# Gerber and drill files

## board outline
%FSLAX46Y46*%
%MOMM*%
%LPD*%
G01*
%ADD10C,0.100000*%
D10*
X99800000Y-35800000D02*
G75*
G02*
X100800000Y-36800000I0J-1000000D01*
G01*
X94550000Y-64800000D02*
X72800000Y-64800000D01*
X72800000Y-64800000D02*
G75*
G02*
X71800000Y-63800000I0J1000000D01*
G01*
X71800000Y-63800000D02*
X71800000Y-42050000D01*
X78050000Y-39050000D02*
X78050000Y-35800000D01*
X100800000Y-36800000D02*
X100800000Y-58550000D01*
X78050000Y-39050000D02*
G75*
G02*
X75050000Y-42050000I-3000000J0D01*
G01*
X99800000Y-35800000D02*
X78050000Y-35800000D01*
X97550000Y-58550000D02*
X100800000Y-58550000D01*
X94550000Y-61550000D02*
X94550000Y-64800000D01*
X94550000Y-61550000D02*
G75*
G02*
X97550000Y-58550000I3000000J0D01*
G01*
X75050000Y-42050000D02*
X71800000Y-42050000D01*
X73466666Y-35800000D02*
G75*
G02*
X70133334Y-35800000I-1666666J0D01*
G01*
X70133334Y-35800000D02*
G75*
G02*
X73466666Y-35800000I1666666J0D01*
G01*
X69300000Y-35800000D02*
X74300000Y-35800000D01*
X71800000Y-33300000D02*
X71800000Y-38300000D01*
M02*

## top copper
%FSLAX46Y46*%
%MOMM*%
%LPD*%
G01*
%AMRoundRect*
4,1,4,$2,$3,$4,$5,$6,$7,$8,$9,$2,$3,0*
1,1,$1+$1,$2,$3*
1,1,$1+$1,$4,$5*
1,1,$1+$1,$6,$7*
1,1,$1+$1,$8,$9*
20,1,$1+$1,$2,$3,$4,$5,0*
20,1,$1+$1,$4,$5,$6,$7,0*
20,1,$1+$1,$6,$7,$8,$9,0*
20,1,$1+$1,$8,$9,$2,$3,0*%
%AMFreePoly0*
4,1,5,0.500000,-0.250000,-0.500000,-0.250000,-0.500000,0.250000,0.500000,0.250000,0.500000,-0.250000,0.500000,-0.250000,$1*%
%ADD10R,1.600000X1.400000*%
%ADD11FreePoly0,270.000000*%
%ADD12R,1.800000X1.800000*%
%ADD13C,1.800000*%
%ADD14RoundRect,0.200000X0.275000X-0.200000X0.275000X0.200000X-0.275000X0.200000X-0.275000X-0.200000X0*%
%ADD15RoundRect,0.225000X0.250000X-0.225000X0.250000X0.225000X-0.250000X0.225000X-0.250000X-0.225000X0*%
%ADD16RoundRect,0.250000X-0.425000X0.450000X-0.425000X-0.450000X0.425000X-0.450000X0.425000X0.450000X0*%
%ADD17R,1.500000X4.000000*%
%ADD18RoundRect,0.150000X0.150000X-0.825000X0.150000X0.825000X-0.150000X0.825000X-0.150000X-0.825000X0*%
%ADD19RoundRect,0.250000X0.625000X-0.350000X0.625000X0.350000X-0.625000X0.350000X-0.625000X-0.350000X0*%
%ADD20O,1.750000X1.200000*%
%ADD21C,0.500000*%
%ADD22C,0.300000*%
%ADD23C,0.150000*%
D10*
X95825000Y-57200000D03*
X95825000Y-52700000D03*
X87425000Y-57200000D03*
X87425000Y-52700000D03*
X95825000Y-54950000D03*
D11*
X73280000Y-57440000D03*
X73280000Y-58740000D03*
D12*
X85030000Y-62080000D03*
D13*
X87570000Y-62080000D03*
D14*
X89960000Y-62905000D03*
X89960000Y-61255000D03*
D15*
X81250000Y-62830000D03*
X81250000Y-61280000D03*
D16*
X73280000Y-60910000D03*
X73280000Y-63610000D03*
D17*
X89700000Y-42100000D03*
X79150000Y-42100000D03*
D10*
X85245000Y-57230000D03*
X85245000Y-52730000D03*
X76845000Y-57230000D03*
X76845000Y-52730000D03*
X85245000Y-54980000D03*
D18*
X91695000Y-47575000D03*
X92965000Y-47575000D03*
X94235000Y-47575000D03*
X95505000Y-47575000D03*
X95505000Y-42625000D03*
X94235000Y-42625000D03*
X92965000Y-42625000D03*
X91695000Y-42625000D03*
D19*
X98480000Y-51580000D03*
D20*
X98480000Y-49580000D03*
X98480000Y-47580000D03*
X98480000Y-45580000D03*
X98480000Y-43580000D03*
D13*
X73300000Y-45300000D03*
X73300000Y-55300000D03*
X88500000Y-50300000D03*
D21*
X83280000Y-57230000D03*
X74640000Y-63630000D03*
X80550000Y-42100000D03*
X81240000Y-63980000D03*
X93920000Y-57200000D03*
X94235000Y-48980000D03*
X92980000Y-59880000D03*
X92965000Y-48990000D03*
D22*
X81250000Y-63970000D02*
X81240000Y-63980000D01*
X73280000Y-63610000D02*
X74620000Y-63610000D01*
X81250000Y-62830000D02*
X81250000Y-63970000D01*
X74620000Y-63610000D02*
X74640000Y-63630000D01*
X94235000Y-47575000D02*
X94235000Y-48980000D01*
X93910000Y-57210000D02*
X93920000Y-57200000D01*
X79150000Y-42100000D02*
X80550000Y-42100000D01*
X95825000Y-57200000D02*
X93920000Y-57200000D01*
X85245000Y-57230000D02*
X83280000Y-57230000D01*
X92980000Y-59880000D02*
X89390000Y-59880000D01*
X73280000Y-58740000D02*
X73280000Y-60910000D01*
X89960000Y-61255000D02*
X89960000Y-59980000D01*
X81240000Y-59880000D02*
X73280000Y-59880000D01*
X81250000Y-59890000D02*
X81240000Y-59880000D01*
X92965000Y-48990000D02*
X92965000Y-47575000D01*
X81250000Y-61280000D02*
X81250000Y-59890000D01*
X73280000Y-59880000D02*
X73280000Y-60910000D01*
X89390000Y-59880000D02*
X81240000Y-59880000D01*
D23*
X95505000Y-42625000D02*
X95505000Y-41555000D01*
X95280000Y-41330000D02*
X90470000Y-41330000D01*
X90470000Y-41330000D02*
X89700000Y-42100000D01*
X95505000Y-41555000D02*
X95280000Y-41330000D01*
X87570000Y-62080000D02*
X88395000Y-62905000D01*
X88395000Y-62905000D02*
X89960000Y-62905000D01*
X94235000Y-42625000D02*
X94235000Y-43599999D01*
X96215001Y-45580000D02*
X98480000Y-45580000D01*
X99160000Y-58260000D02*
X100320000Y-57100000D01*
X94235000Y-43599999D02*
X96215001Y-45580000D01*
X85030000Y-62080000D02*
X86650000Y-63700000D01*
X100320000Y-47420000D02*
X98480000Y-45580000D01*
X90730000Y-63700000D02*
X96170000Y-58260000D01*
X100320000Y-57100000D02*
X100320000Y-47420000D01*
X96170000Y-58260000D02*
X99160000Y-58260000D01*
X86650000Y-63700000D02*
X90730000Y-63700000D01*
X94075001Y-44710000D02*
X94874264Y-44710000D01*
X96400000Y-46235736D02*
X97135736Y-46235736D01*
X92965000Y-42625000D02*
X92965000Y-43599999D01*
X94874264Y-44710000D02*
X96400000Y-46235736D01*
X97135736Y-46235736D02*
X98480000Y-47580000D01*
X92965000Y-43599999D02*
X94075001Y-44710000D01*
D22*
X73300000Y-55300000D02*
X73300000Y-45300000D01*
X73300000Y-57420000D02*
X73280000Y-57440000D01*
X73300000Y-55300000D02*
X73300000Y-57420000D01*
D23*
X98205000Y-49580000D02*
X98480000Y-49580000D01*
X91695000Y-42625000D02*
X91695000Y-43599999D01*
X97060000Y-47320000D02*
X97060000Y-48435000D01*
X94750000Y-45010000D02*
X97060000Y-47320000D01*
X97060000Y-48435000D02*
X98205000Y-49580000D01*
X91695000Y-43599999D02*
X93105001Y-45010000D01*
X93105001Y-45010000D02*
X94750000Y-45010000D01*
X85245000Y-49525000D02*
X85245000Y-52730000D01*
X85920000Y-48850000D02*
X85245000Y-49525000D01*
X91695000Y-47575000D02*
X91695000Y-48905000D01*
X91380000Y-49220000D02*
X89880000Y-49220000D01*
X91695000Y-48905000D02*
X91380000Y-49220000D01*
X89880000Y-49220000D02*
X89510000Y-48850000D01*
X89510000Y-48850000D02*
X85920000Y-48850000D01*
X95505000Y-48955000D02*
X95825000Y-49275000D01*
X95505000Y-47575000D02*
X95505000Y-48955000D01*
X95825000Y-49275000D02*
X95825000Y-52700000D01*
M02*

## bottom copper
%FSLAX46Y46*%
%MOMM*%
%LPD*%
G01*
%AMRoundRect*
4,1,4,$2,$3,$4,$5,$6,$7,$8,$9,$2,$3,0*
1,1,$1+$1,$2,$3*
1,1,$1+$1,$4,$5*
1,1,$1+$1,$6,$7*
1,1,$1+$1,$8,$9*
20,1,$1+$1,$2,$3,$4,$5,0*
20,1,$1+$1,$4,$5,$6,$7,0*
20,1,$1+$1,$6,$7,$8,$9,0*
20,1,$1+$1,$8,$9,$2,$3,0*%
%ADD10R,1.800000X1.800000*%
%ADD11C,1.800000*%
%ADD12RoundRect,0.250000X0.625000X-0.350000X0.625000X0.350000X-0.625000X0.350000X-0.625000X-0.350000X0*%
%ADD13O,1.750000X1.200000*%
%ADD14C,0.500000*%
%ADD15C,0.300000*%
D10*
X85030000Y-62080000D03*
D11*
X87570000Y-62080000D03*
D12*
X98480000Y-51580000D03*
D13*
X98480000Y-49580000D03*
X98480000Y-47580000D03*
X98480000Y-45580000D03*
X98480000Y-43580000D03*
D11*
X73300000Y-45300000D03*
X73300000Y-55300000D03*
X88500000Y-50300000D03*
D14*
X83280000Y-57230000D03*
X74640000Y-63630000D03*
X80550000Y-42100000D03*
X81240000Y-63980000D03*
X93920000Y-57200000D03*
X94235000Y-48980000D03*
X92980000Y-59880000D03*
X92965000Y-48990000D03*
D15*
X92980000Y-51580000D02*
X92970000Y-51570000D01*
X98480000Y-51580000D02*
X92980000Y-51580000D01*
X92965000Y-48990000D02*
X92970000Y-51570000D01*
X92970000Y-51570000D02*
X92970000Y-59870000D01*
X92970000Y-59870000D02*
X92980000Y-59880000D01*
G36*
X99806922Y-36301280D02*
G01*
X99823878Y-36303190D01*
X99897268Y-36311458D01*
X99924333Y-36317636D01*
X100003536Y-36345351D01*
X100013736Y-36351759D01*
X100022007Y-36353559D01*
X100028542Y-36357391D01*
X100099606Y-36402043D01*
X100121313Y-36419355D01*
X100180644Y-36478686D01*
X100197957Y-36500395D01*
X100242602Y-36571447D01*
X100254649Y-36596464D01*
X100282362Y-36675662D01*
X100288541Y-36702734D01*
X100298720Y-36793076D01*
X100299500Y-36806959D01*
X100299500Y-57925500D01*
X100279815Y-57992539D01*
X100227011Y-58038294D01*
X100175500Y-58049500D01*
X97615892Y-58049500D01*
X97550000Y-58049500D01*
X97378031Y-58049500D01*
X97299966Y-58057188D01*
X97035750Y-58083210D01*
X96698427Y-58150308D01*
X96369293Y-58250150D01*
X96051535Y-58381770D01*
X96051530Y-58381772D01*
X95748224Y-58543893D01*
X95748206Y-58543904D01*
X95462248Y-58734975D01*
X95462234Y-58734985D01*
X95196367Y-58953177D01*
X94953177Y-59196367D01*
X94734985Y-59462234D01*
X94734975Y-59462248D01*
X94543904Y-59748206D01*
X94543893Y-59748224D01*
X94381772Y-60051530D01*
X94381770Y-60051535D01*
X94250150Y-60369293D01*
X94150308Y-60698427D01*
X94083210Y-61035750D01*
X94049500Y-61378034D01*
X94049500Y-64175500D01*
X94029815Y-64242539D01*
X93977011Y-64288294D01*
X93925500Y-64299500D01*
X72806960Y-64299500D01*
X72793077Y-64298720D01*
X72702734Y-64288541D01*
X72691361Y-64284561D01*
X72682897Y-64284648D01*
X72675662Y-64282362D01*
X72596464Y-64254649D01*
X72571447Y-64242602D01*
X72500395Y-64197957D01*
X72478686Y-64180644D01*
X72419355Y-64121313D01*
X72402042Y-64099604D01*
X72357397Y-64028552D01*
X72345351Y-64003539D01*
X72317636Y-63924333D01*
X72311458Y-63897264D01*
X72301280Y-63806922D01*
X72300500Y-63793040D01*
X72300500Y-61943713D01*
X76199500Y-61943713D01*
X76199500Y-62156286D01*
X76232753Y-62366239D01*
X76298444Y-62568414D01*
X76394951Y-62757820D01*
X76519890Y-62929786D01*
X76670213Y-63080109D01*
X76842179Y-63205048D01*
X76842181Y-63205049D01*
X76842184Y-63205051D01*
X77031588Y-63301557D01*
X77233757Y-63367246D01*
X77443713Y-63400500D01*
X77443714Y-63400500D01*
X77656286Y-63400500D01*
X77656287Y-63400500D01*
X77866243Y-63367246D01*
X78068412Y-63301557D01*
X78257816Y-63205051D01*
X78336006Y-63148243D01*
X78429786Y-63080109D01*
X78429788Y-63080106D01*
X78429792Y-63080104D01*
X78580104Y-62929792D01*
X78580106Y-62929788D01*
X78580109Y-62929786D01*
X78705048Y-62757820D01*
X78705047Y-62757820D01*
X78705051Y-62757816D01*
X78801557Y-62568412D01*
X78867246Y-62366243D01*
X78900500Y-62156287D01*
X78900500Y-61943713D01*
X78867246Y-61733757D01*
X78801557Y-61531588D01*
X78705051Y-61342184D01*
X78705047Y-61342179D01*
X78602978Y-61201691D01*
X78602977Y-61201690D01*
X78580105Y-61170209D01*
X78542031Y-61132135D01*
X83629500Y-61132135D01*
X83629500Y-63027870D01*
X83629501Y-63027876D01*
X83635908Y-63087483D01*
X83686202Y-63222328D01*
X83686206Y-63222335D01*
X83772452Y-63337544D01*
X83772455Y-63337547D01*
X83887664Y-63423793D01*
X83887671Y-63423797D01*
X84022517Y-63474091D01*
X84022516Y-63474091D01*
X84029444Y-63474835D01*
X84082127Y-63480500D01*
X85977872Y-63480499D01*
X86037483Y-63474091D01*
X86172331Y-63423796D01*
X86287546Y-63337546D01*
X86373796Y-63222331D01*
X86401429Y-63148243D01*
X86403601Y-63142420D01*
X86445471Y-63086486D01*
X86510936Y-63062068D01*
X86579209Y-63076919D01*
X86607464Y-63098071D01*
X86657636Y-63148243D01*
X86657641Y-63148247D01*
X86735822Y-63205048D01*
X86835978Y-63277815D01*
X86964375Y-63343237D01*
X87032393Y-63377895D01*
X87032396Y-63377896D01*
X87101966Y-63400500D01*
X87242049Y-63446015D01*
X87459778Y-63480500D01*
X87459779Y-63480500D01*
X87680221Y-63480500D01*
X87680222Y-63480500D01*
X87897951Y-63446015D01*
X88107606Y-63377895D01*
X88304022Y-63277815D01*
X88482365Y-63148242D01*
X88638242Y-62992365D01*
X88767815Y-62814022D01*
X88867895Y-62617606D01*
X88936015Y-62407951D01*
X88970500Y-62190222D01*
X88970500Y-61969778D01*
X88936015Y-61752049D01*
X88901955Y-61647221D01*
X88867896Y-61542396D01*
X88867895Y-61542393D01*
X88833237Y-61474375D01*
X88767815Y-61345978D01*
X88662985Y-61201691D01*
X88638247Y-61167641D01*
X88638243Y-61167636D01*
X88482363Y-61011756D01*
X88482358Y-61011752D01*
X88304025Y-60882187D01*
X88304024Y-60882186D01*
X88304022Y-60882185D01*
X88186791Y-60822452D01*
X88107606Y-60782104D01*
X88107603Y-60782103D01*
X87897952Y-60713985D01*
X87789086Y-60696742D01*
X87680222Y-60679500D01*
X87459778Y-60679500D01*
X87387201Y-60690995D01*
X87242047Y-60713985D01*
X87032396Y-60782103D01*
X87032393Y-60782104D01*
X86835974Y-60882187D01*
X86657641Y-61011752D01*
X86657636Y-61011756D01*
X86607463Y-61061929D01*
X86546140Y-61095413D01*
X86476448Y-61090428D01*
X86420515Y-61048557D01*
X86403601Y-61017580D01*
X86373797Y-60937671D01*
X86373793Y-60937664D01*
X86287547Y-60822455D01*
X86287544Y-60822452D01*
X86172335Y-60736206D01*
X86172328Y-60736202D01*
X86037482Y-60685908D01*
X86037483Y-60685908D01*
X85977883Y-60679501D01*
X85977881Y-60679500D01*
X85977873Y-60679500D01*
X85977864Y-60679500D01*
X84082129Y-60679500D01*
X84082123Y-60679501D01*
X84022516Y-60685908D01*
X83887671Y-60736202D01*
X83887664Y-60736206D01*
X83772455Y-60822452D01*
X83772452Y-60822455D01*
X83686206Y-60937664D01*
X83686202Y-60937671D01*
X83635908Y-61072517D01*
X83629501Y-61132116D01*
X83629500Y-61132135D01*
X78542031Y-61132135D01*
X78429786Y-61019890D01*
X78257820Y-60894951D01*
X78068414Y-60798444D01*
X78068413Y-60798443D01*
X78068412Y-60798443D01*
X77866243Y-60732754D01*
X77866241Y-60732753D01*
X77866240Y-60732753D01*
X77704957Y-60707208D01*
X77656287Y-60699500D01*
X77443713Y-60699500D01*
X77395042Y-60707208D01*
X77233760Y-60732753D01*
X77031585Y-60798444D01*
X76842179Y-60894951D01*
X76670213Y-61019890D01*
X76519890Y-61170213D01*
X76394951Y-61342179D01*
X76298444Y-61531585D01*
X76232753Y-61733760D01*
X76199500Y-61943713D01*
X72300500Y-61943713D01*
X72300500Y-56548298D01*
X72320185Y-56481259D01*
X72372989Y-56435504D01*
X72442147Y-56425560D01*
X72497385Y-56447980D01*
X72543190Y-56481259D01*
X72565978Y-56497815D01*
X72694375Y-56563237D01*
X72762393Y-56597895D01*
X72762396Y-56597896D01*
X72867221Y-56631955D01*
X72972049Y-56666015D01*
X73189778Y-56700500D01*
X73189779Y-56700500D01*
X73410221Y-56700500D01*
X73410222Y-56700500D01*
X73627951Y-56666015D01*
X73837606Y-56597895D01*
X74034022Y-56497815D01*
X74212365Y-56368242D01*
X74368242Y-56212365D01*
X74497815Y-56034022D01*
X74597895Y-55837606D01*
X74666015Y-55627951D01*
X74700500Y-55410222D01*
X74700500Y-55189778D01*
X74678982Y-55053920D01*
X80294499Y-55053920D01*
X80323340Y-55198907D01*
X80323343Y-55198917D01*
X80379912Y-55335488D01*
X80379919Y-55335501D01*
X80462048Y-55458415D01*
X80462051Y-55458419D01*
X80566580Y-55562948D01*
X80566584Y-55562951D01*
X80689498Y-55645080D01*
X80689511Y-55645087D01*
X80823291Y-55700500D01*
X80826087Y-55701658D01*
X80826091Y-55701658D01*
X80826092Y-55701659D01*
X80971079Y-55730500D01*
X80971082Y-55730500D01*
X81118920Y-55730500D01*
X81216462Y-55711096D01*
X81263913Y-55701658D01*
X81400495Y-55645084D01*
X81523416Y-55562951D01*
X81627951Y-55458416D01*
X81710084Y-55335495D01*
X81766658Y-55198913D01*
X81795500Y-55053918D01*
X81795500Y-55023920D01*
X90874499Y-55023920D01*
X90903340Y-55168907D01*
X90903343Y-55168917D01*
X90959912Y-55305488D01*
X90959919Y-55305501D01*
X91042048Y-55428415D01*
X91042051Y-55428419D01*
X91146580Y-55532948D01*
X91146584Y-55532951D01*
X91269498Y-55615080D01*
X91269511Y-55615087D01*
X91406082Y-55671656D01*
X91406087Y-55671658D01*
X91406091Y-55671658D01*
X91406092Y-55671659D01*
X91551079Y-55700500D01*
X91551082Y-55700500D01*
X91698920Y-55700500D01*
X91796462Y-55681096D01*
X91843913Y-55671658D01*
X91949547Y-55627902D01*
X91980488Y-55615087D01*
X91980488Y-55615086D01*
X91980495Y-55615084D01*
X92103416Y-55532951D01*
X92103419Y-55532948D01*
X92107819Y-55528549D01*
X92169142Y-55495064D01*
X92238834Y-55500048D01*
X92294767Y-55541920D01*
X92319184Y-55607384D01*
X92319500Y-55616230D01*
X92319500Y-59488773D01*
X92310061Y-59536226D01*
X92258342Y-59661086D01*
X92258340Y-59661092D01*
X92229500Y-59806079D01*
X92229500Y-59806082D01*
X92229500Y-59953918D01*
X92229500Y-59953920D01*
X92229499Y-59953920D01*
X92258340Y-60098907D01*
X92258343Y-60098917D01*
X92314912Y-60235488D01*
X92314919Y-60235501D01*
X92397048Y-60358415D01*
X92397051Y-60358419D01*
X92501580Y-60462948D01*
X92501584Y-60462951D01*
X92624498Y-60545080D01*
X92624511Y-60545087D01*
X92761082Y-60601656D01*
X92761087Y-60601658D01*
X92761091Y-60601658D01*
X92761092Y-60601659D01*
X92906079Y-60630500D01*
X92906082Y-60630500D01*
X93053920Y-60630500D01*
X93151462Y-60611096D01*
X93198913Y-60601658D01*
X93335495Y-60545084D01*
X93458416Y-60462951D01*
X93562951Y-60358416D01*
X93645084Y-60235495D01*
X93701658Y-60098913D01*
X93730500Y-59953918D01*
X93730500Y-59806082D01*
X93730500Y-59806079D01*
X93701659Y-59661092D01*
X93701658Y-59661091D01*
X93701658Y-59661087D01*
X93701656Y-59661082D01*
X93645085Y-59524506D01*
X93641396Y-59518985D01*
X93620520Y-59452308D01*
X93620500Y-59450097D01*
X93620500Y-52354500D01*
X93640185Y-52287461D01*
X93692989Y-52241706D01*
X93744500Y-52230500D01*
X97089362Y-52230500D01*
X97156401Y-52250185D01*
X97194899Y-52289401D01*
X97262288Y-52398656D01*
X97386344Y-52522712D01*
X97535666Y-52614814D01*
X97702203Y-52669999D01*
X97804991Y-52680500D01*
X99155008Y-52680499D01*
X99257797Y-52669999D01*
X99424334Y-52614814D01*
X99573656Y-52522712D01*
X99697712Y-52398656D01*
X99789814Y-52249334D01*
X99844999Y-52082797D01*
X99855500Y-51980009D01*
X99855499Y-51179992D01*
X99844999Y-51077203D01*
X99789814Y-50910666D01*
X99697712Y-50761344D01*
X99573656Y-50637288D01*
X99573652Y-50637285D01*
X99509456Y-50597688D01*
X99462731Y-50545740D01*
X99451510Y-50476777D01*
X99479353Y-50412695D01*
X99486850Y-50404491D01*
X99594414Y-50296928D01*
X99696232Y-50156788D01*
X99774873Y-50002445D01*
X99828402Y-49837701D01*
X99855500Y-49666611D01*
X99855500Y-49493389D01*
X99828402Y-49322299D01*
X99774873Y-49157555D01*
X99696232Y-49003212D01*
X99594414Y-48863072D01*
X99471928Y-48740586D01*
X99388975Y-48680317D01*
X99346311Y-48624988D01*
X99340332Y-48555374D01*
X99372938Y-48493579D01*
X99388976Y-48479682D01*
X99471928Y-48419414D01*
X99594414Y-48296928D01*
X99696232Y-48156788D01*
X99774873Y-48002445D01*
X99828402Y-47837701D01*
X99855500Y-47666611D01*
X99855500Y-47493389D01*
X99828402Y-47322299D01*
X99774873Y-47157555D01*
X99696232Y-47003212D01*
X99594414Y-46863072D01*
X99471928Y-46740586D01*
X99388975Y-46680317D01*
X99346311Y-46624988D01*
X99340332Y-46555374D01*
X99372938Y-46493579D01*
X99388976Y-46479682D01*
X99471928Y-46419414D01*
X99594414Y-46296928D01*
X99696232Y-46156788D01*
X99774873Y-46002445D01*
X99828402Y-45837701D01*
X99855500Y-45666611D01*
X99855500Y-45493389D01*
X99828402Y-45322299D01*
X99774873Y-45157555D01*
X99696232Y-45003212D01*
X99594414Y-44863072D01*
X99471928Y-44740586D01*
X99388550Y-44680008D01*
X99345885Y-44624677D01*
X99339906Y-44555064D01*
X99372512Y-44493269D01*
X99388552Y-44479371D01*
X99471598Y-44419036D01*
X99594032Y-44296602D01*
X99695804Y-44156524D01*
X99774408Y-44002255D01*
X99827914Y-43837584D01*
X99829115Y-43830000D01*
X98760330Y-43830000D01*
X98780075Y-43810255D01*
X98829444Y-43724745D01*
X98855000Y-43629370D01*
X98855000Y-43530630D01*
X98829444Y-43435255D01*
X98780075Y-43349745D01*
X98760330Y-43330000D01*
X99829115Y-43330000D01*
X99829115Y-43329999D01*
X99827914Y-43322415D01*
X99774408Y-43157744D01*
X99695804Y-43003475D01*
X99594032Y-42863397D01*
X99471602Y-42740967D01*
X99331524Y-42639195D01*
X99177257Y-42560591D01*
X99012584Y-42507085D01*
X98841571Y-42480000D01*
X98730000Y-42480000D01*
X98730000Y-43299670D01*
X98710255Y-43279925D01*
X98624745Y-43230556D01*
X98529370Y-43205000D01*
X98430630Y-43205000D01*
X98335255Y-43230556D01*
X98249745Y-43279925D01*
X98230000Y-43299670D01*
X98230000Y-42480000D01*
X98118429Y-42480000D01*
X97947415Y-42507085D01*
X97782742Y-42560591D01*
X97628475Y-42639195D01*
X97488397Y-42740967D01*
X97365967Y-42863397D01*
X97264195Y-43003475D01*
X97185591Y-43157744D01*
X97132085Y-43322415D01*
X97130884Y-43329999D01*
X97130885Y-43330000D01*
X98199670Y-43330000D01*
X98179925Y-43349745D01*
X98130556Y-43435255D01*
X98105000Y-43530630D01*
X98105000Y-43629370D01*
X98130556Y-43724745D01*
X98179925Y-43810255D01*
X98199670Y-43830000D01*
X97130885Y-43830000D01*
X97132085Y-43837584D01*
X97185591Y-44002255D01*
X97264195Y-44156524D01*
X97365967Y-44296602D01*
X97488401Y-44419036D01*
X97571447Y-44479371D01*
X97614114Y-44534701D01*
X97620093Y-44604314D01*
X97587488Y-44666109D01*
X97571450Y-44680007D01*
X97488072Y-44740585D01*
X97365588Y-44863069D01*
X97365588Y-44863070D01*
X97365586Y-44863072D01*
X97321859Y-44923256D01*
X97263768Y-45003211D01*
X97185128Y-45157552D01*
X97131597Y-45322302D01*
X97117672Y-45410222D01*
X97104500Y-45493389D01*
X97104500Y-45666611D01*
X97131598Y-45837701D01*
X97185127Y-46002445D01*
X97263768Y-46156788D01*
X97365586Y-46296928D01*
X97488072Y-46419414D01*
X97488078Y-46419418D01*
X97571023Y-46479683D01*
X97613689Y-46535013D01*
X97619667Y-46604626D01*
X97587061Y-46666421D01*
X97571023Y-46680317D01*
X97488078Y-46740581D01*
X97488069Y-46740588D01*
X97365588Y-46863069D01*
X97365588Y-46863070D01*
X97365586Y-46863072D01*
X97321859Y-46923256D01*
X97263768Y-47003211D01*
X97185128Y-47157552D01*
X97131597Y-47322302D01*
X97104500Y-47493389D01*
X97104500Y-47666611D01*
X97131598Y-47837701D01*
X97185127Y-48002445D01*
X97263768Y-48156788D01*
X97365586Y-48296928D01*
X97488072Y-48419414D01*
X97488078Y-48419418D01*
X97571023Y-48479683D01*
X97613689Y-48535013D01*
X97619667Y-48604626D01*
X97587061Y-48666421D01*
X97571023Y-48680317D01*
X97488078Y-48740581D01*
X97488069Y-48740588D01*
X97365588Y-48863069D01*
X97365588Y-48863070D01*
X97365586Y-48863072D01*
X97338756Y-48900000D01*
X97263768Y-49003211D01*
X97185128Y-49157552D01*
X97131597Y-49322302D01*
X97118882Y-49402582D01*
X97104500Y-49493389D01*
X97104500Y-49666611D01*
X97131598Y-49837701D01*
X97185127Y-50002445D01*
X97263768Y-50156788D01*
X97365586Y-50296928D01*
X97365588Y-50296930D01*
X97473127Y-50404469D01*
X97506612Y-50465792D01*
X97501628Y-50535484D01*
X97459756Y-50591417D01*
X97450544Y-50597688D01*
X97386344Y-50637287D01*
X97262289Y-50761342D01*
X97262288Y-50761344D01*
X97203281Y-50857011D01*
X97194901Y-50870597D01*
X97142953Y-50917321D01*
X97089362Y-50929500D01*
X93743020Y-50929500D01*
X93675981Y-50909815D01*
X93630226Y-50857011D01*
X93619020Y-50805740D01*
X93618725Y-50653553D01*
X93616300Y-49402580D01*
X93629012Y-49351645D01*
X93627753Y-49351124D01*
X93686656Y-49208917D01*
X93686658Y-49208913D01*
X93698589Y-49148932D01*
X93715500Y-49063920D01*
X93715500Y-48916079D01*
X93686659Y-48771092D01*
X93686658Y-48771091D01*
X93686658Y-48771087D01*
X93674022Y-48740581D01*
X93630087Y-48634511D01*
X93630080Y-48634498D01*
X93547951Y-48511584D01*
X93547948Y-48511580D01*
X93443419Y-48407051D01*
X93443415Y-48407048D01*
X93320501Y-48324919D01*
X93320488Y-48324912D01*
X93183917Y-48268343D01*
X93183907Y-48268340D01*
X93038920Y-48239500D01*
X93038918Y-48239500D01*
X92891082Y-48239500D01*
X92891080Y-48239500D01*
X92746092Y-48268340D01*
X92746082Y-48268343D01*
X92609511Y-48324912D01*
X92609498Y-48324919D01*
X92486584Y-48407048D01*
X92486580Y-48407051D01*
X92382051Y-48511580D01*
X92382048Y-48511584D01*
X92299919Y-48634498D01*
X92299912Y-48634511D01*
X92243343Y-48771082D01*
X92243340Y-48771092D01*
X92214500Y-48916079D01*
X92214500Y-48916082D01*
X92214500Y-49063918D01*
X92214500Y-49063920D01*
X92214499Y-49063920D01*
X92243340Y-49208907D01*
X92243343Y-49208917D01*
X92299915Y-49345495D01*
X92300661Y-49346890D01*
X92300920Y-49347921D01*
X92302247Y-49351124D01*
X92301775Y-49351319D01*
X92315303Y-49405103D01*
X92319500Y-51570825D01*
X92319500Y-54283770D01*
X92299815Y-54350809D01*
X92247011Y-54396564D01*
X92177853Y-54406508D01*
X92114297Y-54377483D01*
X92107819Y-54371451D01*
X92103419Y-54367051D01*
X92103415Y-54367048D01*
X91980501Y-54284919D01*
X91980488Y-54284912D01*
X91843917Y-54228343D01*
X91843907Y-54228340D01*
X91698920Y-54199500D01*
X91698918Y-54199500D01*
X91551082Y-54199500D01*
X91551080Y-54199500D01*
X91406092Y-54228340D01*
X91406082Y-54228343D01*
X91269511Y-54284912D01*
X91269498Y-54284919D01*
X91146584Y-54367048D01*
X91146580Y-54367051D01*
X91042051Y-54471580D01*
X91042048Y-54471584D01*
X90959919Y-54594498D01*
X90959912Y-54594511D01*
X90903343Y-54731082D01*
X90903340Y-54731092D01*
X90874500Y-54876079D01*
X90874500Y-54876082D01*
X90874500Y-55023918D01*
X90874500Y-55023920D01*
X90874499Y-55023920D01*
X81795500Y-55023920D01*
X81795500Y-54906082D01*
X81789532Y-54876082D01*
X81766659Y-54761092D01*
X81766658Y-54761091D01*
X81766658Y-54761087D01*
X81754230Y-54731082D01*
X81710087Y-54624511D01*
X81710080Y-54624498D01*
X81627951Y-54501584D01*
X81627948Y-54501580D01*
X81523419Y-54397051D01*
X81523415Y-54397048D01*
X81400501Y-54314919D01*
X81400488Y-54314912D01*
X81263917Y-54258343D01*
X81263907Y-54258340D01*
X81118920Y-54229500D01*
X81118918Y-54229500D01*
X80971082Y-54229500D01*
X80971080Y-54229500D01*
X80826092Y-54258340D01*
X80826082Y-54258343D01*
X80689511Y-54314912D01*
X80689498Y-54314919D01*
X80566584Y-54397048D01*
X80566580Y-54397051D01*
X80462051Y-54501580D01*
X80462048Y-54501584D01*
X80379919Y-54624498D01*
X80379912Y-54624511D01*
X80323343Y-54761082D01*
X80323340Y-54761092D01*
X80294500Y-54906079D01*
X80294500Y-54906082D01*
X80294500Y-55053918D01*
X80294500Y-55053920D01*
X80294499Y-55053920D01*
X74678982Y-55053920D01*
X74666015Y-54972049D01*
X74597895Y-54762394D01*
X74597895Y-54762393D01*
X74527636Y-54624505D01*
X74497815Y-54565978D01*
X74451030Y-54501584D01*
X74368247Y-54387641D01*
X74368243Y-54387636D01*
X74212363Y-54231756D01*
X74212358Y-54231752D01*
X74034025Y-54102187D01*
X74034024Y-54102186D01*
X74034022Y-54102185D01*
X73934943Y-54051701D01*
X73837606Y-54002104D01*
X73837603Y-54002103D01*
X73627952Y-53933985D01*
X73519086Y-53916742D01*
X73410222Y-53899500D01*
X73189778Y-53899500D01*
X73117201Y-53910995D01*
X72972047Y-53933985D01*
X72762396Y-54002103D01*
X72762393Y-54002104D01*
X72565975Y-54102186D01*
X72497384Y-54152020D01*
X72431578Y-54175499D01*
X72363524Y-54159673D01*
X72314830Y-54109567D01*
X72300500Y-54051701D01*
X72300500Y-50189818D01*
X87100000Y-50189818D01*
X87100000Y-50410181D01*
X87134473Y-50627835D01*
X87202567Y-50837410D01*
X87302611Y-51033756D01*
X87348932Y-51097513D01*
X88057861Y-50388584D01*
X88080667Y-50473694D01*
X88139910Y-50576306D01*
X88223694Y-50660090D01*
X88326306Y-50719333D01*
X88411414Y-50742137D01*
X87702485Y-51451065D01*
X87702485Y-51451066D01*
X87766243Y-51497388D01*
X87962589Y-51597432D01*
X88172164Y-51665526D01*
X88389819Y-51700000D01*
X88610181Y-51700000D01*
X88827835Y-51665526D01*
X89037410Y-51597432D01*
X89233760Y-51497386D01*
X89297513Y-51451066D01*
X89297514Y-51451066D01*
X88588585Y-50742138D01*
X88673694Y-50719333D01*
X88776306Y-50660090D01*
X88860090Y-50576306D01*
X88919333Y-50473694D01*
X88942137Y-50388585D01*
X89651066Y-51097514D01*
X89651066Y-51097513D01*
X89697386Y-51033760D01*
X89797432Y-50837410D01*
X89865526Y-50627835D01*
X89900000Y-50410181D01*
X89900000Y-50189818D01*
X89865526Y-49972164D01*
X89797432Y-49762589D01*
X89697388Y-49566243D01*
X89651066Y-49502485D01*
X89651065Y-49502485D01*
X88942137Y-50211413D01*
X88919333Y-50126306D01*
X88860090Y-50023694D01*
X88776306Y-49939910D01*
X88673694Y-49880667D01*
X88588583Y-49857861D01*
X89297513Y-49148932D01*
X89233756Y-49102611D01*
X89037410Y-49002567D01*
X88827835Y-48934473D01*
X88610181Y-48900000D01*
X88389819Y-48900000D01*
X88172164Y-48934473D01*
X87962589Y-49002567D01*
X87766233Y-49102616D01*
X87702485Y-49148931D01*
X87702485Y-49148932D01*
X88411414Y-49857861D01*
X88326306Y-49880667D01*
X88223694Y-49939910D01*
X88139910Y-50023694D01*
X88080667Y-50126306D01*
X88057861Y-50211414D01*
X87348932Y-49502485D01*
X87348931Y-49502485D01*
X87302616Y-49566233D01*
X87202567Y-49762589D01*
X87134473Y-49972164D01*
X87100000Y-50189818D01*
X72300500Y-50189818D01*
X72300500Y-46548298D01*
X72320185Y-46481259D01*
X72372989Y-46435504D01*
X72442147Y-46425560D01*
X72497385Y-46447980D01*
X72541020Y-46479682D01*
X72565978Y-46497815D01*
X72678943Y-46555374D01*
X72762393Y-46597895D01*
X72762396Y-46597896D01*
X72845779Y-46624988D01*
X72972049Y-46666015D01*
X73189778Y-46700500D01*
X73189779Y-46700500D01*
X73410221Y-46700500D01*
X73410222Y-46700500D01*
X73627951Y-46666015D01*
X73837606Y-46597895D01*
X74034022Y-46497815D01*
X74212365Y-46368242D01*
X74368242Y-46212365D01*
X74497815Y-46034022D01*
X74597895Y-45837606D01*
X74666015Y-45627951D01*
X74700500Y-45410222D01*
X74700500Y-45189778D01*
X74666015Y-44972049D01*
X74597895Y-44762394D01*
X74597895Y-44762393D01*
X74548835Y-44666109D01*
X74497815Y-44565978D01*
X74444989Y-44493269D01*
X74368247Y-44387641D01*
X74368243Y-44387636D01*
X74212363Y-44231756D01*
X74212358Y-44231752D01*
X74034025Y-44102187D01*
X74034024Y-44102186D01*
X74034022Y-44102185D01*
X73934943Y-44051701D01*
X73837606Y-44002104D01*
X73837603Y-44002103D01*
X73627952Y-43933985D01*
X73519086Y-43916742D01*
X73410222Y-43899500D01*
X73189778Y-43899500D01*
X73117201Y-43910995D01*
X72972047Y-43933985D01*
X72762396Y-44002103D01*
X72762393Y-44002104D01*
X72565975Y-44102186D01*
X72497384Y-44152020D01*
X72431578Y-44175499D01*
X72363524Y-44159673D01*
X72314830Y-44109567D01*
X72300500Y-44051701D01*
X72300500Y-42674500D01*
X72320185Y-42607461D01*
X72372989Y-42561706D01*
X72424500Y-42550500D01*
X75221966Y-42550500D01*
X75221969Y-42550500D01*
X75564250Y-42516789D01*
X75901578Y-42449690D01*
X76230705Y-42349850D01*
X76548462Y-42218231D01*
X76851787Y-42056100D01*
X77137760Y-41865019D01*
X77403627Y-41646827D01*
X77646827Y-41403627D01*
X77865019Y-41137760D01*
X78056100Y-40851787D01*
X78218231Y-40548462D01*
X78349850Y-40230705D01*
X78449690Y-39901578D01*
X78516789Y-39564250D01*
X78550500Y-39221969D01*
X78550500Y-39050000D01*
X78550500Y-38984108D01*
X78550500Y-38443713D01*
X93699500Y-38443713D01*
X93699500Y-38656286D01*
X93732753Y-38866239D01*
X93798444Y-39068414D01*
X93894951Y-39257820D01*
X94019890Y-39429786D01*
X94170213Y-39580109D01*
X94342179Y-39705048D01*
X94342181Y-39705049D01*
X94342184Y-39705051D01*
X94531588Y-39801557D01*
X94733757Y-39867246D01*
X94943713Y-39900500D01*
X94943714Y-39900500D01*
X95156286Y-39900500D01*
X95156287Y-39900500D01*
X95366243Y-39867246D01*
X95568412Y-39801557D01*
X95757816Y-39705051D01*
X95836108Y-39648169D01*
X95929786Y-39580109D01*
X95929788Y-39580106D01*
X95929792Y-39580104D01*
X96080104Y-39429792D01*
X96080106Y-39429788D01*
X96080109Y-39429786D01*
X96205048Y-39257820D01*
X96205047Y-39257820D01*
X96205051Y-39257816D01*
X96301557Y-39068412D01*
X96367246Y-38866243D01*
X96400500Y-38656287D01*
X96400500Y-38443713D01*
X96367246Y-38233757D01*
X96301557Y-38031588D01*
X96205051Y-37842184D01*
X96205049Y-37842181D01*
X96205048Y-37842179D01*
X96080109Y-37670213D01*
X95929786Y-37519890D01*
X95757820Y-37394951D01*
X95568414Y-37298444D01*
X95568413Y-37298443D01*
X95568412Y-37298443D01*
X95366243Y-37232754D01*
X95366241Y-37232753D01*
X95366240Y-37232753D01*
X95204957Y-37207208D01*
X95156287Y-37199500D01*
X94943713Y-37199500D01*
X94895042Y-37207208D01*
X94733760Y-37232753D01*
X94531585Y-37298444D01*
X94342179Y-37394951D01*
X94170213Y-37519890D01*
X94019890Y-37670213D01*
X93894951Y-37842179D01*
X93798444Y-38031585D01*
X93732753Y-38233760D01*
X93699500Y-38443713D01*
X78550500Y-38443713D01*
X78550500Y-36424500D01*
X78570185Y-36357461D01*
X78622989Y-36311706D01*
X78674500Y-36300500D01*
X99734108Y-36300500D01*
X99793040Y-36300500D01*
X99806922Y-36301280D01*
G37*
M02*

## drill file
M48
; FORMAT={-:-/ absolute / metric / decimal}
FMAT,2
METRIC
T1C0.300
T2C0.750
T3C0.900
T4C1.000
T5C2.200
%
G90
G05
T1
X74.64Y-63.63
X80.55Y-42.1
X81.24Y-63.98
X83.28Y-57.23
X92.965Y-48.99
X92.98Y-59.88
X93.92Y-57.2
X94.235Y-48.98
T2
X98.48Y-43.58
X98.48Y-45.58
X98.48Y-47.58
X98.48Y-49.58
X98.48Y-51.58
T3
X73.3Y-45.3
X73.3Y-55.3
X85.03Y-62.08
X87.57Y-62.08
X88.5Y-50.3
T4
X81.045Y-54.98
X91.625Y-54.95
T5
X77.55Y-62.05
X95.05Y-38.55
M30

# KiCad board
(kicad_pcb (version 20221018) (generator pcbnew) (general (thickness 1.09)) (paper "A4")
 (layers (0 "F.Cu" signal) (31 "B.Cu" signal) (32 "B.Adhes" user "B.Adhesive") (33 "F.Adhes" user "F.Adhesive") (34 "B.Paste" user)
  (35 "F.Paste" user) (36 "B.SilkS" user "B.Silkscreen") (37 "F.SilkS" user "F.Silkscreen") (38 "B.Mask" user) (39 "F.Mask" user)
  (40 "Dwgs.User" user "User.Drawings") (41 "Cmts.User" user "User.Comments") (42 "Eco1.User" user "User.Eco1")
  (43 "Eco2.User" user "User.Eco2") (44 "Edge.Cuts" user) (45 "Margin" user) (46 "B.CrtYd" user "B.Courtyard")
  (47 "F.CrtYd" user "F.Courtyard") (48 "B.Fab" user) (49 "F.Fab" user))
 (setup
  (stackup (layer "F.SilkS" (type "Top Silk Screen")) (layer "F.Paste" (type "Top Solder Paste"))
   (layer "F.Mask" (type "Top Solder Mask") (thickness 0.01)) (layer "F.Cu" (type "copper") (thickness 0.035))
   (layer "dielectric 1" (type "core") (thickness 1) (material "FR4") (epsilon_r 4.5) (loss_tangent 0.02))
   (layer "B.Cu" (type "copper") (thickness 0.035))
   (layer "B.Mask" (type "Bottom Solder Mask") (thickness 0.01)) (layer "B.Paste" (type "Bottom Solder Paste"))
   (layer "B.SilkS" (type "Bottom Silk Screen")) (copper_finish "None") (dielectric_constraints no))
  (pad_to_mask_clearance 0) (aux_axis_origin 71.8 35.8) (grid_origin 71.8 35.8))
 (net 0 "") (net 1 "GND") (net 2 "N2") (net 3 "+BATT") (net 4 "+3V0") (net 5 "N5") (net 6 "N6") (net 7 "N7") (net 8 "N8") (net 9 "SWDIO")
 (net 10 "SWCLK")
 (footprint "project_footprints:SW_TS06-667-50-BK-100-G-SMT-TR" (layer "F.Cu") (at 91.625 54.95 180)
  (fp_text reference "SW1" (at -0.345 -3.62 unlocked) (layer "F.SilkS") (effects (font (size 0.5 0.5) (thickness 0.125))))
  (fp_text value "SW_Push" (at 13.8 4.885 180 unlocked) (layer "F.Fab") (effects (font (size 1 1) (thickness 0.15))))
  (pad "1" smd rect (at -4.2 -2.25 180) (size 1.6 1.4) (layers "F.Cu" "F.Paste" "F.Mask") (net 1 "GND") (solder_mask_margin 0.102))
  (pad "2" smd rect (at -4.2 2.25 180) (size 1.6 1.4) (layers "F.Cu" "F.Paste" "F.Mask") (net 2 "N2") (solder_mask_margin 0.102))
  (pad "3" smd rect (at 4.2 -2.25 180) (size 1.6 1.4) (layers "F.Cu" "F.Paste" "F.Mask") (solder_mask_margin 0.102))
  (pad "4" smd rect (at 4.2 2.25 180) (size 1.6 1.4) (layers "F.Cu" "F.Paste" "F.Mask") (solder_mask_margin 0.102))
  (pad "5" smd rect (at -4.2 0 180) (size 1.6 1.4) (layers "F.Cu" "F.Paste" "F.Mask") (solder_mask_margin 0.102)))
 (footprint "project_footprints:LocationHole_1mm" (layer "F.Cu") (at 81.045 54.98)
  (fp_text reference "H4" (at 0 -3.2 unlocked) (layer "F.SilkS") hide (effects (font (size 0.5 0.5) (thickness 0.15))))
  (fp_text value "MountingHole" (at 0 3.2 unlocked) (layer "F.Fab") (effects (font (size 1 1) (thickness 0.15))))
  (pad "" np_thru_hole circle (at 0 0) (size 1 1) (drill 1) (layers "F&B.Cu" "*.Mask")))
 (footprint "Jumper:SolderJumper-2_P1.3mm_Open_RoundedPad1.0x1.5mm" (layer "F.Cu") (at 73.28 58.09 -90) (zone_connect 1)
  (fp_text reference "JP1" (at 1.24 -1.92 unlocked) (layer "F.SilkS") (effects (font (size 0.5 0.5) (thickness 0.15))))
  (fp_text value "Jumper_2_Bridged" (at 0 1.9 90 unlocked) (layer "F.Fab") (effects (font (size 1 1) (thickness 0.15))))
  (pad "1" smd custom (at -0.65 0 270) (size 1 0.5) (layers "F.Cu" "F.Mask") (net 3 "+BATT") (zone_connect 2) (thermal_bridge_angle 45)
   (options (clearance outline) (anchor rect)) (primitives))
  (pad "2" smd custom (at 0.65 0 270) (size 1 0.5) (layers "F.Cu" "F.Mask") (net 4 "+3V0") (zone_connect 2) (thermal_bridge_angle 45)
   (options (clearance outline) (anchor rect)) (primitives)))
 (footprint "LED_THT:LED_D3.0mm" (layer "F.Cu") (at 85.03 62.08)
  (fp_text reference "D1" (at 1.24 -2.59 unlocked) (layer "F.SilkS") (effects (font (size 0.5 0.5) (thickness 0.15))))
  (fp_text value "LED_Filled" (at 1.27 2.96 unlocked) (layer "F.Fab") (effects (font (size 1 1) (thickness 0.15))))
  (pad "1" thru_hole rect (at 0 0) (size 1.8 1.8) (drill 0.9) (layers "*.Cu" "*.Mask") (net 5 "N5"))
  (pad "2" thru_hole circle (at 2.54 0) (size 1.8 1.8) (drill 0.9) (layers "*.Cu" "*.Mask") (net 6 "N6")))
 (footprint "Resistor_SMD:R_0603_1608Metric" (layer "F.Cu") (at 89.96 62.08 90)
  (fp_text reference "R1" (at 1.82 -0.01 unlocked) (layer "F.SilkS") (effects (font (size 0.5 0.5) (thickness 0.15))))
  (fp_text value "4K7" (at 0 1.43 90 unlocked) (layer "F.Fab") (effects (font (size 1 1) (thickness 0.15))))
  (pad "1" smd roundrect (at -0.825 0 90) (size 0.8 0.95) (layers "F.Cu" "F.Paste" "F.Mask") (roundrect_rratio 0.25) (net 6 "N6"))
  (pad "2" smd roundrect (at 0.825 0 90) (size 0.8 0.95) (layers "F.Cu" "F.Paste" "F.Mask") (roundrect_rratio 0.25) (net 4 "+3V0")))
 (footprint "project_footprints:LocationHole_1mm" (layer "F.Cu") (at 91.625 54.95)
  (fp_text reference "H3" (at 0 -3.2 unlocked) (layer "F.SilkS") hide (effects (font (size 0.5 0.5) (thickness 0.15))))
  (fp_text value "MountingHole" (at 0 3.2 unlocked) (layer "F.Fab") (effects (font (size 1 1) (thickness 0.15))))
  (pad "" np_thru_hole circle (at 0 0) (size 1 1) (drill 1) (layers "F&B.Cu" "*.Mask")))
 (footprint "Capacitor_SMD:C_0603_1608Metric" (layer "F.Cu") (at 81.25 62.055 90)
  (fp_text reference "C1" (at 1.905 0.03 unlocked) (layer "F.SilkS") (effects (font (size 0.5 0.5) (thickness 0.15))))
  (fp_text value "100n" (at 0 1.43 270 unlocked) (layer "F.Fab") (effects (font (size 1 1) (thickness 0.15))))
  (pad "1" smd roundrect (at -0.775 0 90) (size 0.9 0.95) (layers "F.Cu" "F.Paste" "F.Mask") (roundrect_rratio 0.25) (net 1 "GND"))
  (pad "2" smd roundrect (at 0.775 0 90) (size 0.9 0.95) (layers "F.Cu" "F.Paste" "F.Mask") (roundrect_rratio 0.25) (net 4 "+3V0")))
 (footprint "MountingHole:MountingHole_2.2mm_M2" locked (layer "F.Cu") (at 77.55 62.05)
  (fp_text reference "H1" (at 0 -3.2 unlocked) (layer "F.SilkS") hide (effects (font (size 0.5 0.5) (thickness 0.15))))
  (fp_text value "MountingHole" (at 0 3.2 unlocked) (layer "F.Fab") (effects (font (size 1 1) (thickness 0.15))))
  (pad "" np_thru_hole circle locked (at 0 0) (size 2.2 2.2) (drill 2.2) (layers "*.Cu" "*.Mask")))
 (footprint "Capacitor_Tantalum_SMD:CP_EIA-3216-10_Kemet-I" (layer "F.Cu") (at 73.28 62.26 -90)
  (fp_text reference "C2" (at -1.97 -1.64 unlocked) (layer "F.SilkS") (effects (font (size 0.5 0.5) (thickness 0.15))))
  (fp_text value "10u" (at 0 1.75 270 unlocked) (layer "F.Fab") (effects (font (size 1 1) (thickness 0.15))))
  (pad "1" smd roundrect (at -1.35 0 270) (size 1.4 1.35) (layers "F.Cu" "F.Paste" "F.Mask") (roundrect_rratio 0.1851851852) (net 4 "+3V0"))
  (pad "2" smd roundrect (at 1.35 0 270) (size 1.4 1.35) (layers "F.Cu" "F.Paste" "F.Mask") (roundrect_rratio 0.1851851852) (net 1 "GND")))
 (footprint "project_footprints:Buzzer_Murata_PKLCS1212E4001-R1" (layer "F.Cu") (at 84.4 42.1 180)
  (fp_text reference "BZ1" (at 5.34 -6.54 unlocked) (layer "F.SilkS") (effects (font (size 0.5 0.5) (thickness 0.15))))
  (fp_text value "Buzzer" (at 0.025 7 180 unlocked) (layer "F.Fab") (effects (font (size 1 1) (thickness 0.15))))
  (pad "1" smd rect (at -5.3 0 180) (size 1.5 4) (layers "F.Cu" "F.Paste" "F.Mask") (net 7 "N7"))
  (pad "2" smd rect (at 5.25 0 180) (size 1.5 4) (layers "F.Cu" "F.Paste" "F.Mask") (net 1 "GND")))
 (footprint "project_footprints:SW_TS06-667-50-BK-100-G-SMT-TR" (layer "F.Cu") (at 81.045 54.98 180)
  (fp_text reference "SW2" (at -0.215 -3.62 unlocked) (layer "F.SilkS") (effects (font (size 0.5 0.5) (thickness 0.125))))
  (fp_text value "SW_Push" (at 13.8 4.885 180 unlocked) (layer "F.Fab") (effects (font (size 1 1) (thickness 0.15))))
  (pad "1" smd rect (at -4.2 -2.25 180) (size 1.6 1.4) (layers "F.Cu" "F.Paste" "F.Mask") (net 1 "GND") (solder_mask_margin 0.102))
  (pad "2" smd rect (at -4.2 2.25 180) (size 1.6 1.4) (layers "F.Cu" "F.Paste" "F.Mask") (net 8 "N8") (solder_mask_margin 0.102))
  (pad "3" smd rect (at 4.2 -2.25 180) (size 1.6 1.4) (layers "F.Cu" "F.Paste" "F.Mask") (solder_mask_margin 0.102))
  (pad "4" smd rect (at 4.2 2.25 180) (size 1.6 1.4) (layers "F.Cu" "F.Paste" "F.Mask") (solder_mask_margin 0.102))
  (pad "5" smd rect (at -4.2 0 180) (size 1.6 1.4) (layers "F.Cu" "F.Paste" "F.Mask") (solder_mask_margin 0.102)))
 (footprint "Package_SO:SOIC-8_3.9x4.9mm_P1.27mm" (layer "F.Cu") (at 93.6 45.1 90)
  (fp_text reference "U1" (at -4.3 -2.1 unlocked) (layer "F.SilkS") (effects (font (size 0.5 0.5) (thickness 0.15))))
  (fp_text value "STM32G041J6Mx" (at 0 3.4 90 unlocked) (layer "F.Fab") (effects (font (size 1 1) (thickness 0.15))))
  (pad "1" smd roundrect (at -2.475 -1.905 90) (size 1.95 0.6) (layers "F.Cu" "F.Paste" "F.Mask") (roundrect_rratio 0.25) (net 8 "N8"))
  (pad "2" smd roundrect (at -2.475 -0.635 90) (size 1.95 0.6) (layers "F.Cu" "F.Paste" "F.Mask") (roundrect_rratio 0.25) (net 4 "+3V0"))
  (pad "3" smd roundrect (at -2.475 0.635 90) (size 1.95 0.6) (layers "F.Cu" "F.Paste" "F.Mask") (roundrect_rratio 0.25) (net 1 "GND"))
  (pad "4" smd roundrect (at -2.475 1.905 90) (size 1.95 0.6) (layers "F.Cu" "F.Paste" "F.Mask") (roundrect_rratio 0.25) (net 2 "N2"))
  (pad "5" smd roundrect (at 2.475 1.905 90) (size 1.95 0.6) (layers "F.Cu" "F.Paste" "F.Mask") (roundrect_rratio 0.25) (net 7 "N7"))
  (pad "6" smd roundrect (at 2.475 0.635 90) (size 1.95 0.6) (layers "F.Cu" "F.Paste" "F.Mask") (roundrect_rratio 0.25) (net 5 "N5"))
  (pad "7" smd roundrect (at 2.475 -0.635 90) (size 1.95 0.6) (layers "F.Cu" "F.Paste" "F.Mask") (roundrect_rratio 0.25) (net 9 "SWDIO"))
  (pad "8" smd roundrect (at 2.475 -1.905 90) (size 1.95 0.6) (layers "F.Cu" "F.Paste" "F.Mask") (roundrect_rratio 0.25) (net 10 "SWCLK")))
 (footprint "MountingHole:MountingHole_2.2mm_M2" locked (layer "F.Cu") (at 95.05 38.55)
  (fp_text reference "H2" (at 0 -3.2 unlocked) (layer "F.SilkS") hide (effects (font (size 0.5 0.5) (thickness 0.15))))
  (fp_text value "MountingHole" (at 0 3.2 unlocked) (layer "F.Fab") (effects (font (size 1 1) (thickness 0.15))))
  (pad "" np_thru_hole circle locked (at 0 0) (size 2.2 2.2) (drill 2.2) (layers "*.Cu" "*.Mask")))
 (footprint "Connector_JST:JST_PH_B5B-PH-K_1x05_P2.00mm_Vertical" (layer "B.Cu") (at 98.48 51.58 90)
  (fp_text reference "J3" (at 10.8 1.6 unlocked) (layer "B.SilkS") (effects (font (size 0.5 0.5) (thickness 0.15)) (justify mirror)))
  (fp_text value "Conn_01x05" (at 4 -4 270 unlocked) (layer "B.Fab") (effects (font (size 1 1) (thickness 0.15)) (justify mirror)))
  (pad "1" thru_hole roundrect (at 0 0 90) (size 1.2 1.75) (drill 0.75) (layers "*.Cu" "*.Mask") (roundrect_rratio 0.2083333333)
   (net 4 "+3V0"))
  (pad "2" thru_hole oval (at 2 0 90) (size 1.2 1.75) (drill 0.75) (layers "*.Cu" "*.Mask") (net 10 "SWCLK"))
  (pad "3" thru_hole oval (at 4 0 90) (size 1.2 1.75) (drill 0.75) (layers "*.Cu" "*.Mask") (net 9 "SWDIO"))
  (pad "4" thru_hole oval (at 6 0 90) (size 1.2 1.75) (drill 0.75) (layers "*.Cu" "*.Mask") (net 5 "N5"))
  (pad "5" thru_hole oval (at 8 0 90) (size 1.2 1.75) (drill 0.75) (layers "*.Cu" "*.Mask") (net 1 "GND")))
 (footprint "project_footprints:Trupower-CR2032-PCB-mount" (layer "B.Cu") (at 83.3 50.3)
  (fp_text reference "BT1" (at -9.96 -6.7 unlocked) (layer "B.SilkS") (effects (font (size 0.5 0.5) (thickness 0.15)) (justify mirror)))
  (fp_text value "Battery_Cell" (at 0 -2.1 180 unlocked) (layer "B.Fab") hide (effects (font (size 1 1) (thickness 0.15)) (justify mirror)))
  (pad "1" thru_hole circle (at -10 -5 90) (size 1.8 1.8) (drill 0.9) (layers "*.Cu" "*.Mask") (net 3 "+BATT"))
  (pad "1" thru_hole circle (at -10 5 90) (size 1.8 1.8) (drill 0.9) (layers "*.Cu" "*.Mask") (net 3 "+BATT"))
  (pad "2" thru_hole circle (at 5.2 0 90) (size 1.8 1.8) (drill 0.9) (layers "*.Cu" "*.Mask") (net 1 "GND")))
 (gr_arc (start 99.8 35.8) (mid 100.507107 36.092893) (end 100.8 36.8) (stroke (width 0.1) (type solid)) (layer "Edge.Cuts"))
 (gr_line (start 94.55 64.8) (end 72.8 64.8) (stroke (width 0.1) (type solid)) (layer "Edge.Cuts"))
 (gr_arc (start 72.8 64.8) (mid 72.092893 64.507107) (end 71.8 63.8) (stroke (width 0.1) (type solid)) (layer "Edge.Cuts"))
 (gr_line (start 71.8 63.8) (end 71.8 42.05) (stroke (width 0.1) (type solid)) (layer "Edge.Cuts"))
 (gr_line (start 78.05 39.05) (end 78.05 35.8) (stroke (width 0.1) (type solid)) (layer "Edge.Cuts"))
 (gr_line (start 100.8 36.8) (end 100.8 58.55) (stroke (width 0.1) (type solid)) (layer "Edge.Cuts"))
 (gr_arc (start 78.05 39.05) (mid 77.17132 41.17132) (end 75.05 42.05) (stroke (width 0.1) (type solid)) (layer "Edge.Cuts"))
 (gr_line (start 99.8 35.8) (end 78.05 35.8) (stroke (width 0.1) (type solid)) (layer "Edge.Cuts"))
 (gr_line (start 97.55 58.55) (end 100.8 58.55) (stroke (width 0.1) (type solid)) (layer "Edge.Cuts"))
 (gr_line (start 94.55 61.55) (end 94.55 64.8) (stroke (width 0.1) (type solid)) (layer "Edge.Cuts"))
 (gr_arc (start 94.55 61.55) (mid 95.42868 59.42868) (end 97.55 58.55) (stroke (width 0.1) (type solid)) (layer "Edge.Cuts"))
 (gr_line (start 75.05 42.05) (end 71.8 42.05) (stroke (width 0.1) (type solid)) (layer "Edge.Cuts"))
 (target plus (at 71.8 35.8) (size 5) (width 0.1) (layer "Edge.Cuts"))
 (segment (start 81.25 63.97) (end 81.24 63.98) (width 0.3) (layer "F.Cu") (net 1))
 (segment (start 73.28 63.61) (end 74.62 63.61) (width 0.3) (layer "F.Cu") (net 1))
 (segment (start 81.25 62.83) (end 81.25 63.97) (width 0.3) (layer "F.Cu") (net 1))
 (segment (start 74.62 63.61) (end 74.64 63.63) (width 0.3) (layer "F.Cu") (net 1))
 (segment (start 94.235 47.575) (end 94.235 48.98) (width 0.3) (layer "F.Cu") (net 1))
 (segment (start 93.91 57.21) (end 93.92 57.2) (width 0.3) (layer "F.Cu") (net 1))
 (segment (start 79.15 42.1) (end 80.55 42.1) (width 0.3) (layer "F.Cu") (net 1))
 (segment (start 95.825 57.2) (end 93.92 57.2) (width 0.3) (layer "F.Cu") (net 1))
 (segment (start 85.245 57.23) (end 83.28 57.23) (width 0.3) (layer "F.Cu") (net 1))
 (via (at 83.28 57.23) (size 0.5) (drill 0.3) (layers "F.Cu" "B.Cu") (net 1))
 (via (at 74.64 63.63) (size 0.5) (drill 0.3) (layers "F.Cu" "B.Cu") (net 1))
 (via (at 80.55 42.1) (size 0.5) (drill 0.3) (layers "F.Cu" "B.Cu") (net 1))
 (via (at 81.24 63.98) (size 0.5) (drill 0.3) (layers "F.Cu" "B.Cu") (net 1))
 (via (at 93.92 57.2) (size 0.5) (drill 0.3) (layers "F.Cu" "B.Cu") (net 1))
 (via (at 94.235 48.98) (size 0.5) (drill 0.3) (layers "F.Cu" "B.Cu") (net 1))
 (segment (start 92.98 59.88) (end 89.39 59.88) (width 0.3) (layer "F.Cu") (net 4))
 (segment (start 73.28 58.74) (end 73.28 60.91) (width 0.3) (layer "F.Cu") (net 4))
 (segment (start 89.96 61.255) (end 89.96 59.98) (width 0.3) (layer "F.Cu") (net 4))
 (segment (start 81.24 59.88) (end 73.28 59.88) (width 0.3) (layer "F.Cu") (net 4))
 (segment (start 81.25 59.89) (end 81.24 59.88) (width 0.3) (layer "F.Cu") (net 4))
 (segment (start 92.965 48.99) (end 92.965 47.575) (width 0.3) (layer "F.Cu") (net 4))
 (segment (start 81.25 61.28) (end 81.25 59.89) (width 0.3) (layer "F.Cu") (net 4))
 (segment (start 73.28 59.88) (end 73.28 60.91) (width 0.3) (layer "F.Cu") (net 4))
 (segment (start 89.39 59.88) (end 81.24 59.88) (width 0.3) (layer "F.Cu") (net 4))
 (via (at 92.98 59.88) (size 0.5) (drill 0.3) (layers "F.Cu" "B.Cu") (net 4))
 (via (at 92.965 48.99) (size 0.5) (drill 0.3) (layers "F.Cu" "B.Cu") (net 4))
 (segment (start 92.98 51.58) (end 92.97 51.57) (width 0.3) (layer "B.Cu") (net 4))
 (segment (start 98.48 51.58) (end 92.98 51.58) (width 0.3) (layer "B.Cu") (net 4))
 (segment (start 92.965 48.99) (end 92.97 51.57) (width 0.3) (layer "B.Cu") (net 4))
 (segment (start 92.97 51.57) (end 92.97 59.87) (width 0.3) (layer "B.Cu") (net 4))
 (segment (start 92.97 59.87) (end 92.98 59.88) (width 0.3) (layer "B.Cu") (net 4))
 (segment (start 95.505 42.625) (end 95.505 41.555) (width 0.15) (layer "F.Cu") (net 7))
 (segment (start 95.28 41.33) (end 90.47 41.33) (width 0.15) (layer "F.Cu") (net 7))
 (segment (start 90.47 41.33) (end 89.7 42.1) (width 0.15) (layer "F.Cu") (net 7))
 (segment (start 95.505 41.555) (end 95.28 41.33) (width 0.15) (layer "F.Cu") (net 7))
 (segment (start 87.57 62.08) (end 88.395 62.905) (width 0.15) (layer "F.Cu") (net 6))
 (segment (start 88.395 62.905) (end 89.96 62.905) (width 0.15) (layer "F.Cu") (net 6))
 (segment (start 94.235 42.625) (end 94.235 43.599999) (width 0.15) (layer "F.Cu") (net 5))
 (segment (start 96.215001 45.58) (end 98.48 45.58) (width 0.15) (layer "F.Cu") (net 5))
 (segment (start 99.16 58.26) (end 100.32 57.1) (width 0.15) (layer "F.Cu") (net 5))
 (segment (start 94.235 43.599999) (end 96.215001 45.58) (width 0.15) (layer "F.Cu") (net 5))
 (segment (start 85.03 62.08) (end 86.65 63.7) (width 0.15) (layer "F.Cu") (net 5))
 (segment (start 100.32 47.42) (end 98.48 45.58) (width 0.15) (layer "F.Cu") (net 5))
 (segment (start 90.73 63.7) (end 96.17 58.26) (width 0.15) (layer "F.Cu") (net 5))
 (segment (start 100.32 57.1) (end 100.32 47.42) (width 0.15) (layer "F.Cu") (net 5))
 (segment (start 96.17 58.26) (end 99.16 58.26) (width 0.15) (layer "F.Cu") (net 5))
 (segment (start 86.65 63.7) (end 90.73 63.7) (width 0.15) (layer "F.Cu") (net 5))
 (segment (start 94.075001 44.71) (end 94.874264 44.71) (width 0.15) (layer "F.Cu") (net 9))
 (segment (start 96.4 46.235736) (end 97.135736 46.235736) (width 0.15) (layer "F.Cu") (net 9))
 (segment (start 92.965 42.625) (end 92.965 43.599999) (width 0.15) (layer "F.Cu") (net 9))
 (segment (start 94.874264 44.71) (end 96.4 46.235736) (width 0.15) (layer "F.Cu") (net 9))
 (segment (start 97.135736 46.235736) (end 98.48 47.58) (width 0.15) (layer "F.Cu") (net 9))
 (segment (start 92.965 43.599999) (end 94.075001 44.71) (width 0.15) (layer "F.Cu") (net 9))
 (segment (start 73.3 55.3) (end 73.3 45.3) (width 0.3) (layer "F.Cu") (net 3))
 (segment (start 73.3 57.42) (end 73.28 57.44) (width 0.3) (layer "F.Cu") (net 3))
 (segment (start 73.3 55.3) (end 73.3 57.42) (width 0.3) (layer "F.Cu") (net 3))
 (segment (start 98.205 49.58) (end 98.48 49.58) (width 0.15) (layer "F.Cu") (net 10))
 (segment (start 91.695 42.625) (end 91.695 43.599999) (width 0.15) (layer "F.Cu") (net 10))
 (segment (start 97.06 47.32) (end 97.06 48.435) (width 0.15) (layer "F.Cu") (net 10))
 (segment (start 94.75 45.01) (end 97.06 47.32) (width 0.15) (layer "F.Cu") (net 10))
 (segment (start 97.06 48.435) (end 98.205 49.58) (width 0.15) (layer "F.Cu") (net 10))
 (segment (start 91.695 43.599999) (end 93.105001 45.01) (width 0.15) (layer "F.Cu") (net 10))
 (segment (start 93.105001 45.01) (end 94.75 45.01) (width 0.15) (layer "F.Cu") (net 10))
 (segment (start 85.245 49.525) (end 85.245 52.73) (width 0.15) (layer "F.Cu") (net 8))
 (segment (start 85.92 48.85) (end 85.245 49.525) (width 0.15) (layer "F.Cu") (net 8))
 (segment (start 91.695 47.575) (end 91.695 48.905) (width 0.15) (layer "F.Cu") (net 8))
 (segment (start 91.38 49.22) (end 89.88 49.22) (width 0.15) (layer "F.Cu") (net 8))
 (segment (start 91.695 48.905) (end 91.38 49.22) (width 0.15) (layer "F.Cu") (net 8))
 (segment (start 89.88 49.22) (end 89.51 48.85) (width 0.15) (layer "F.Cu") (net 8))
 (segment (start 89.51 48.85) (end 85.92 48.85) (width 0.15) (layer "F.Cu") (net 8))
 (segment (start 95.505 48.955) (end 95.825 49.275) (width 0.15) (layer "F.Cu") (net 2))
 (segment (start 95.505 47.575) (end 95.505 48.955) (width 0.15) (layer "F.Cu") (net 2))
 (segment (start 95.825 49.275) (end 95.825 52.7) (width 0.15) (layer "F.Cu") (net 2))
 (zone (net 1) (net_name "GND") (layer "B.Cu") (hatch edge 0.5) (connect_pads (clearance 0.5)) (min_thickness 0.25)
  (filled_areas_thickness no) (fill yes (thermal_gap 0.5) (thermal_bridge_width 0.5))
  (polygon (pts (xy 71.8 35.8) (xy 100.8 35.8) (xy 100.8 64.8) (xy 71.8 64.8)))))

